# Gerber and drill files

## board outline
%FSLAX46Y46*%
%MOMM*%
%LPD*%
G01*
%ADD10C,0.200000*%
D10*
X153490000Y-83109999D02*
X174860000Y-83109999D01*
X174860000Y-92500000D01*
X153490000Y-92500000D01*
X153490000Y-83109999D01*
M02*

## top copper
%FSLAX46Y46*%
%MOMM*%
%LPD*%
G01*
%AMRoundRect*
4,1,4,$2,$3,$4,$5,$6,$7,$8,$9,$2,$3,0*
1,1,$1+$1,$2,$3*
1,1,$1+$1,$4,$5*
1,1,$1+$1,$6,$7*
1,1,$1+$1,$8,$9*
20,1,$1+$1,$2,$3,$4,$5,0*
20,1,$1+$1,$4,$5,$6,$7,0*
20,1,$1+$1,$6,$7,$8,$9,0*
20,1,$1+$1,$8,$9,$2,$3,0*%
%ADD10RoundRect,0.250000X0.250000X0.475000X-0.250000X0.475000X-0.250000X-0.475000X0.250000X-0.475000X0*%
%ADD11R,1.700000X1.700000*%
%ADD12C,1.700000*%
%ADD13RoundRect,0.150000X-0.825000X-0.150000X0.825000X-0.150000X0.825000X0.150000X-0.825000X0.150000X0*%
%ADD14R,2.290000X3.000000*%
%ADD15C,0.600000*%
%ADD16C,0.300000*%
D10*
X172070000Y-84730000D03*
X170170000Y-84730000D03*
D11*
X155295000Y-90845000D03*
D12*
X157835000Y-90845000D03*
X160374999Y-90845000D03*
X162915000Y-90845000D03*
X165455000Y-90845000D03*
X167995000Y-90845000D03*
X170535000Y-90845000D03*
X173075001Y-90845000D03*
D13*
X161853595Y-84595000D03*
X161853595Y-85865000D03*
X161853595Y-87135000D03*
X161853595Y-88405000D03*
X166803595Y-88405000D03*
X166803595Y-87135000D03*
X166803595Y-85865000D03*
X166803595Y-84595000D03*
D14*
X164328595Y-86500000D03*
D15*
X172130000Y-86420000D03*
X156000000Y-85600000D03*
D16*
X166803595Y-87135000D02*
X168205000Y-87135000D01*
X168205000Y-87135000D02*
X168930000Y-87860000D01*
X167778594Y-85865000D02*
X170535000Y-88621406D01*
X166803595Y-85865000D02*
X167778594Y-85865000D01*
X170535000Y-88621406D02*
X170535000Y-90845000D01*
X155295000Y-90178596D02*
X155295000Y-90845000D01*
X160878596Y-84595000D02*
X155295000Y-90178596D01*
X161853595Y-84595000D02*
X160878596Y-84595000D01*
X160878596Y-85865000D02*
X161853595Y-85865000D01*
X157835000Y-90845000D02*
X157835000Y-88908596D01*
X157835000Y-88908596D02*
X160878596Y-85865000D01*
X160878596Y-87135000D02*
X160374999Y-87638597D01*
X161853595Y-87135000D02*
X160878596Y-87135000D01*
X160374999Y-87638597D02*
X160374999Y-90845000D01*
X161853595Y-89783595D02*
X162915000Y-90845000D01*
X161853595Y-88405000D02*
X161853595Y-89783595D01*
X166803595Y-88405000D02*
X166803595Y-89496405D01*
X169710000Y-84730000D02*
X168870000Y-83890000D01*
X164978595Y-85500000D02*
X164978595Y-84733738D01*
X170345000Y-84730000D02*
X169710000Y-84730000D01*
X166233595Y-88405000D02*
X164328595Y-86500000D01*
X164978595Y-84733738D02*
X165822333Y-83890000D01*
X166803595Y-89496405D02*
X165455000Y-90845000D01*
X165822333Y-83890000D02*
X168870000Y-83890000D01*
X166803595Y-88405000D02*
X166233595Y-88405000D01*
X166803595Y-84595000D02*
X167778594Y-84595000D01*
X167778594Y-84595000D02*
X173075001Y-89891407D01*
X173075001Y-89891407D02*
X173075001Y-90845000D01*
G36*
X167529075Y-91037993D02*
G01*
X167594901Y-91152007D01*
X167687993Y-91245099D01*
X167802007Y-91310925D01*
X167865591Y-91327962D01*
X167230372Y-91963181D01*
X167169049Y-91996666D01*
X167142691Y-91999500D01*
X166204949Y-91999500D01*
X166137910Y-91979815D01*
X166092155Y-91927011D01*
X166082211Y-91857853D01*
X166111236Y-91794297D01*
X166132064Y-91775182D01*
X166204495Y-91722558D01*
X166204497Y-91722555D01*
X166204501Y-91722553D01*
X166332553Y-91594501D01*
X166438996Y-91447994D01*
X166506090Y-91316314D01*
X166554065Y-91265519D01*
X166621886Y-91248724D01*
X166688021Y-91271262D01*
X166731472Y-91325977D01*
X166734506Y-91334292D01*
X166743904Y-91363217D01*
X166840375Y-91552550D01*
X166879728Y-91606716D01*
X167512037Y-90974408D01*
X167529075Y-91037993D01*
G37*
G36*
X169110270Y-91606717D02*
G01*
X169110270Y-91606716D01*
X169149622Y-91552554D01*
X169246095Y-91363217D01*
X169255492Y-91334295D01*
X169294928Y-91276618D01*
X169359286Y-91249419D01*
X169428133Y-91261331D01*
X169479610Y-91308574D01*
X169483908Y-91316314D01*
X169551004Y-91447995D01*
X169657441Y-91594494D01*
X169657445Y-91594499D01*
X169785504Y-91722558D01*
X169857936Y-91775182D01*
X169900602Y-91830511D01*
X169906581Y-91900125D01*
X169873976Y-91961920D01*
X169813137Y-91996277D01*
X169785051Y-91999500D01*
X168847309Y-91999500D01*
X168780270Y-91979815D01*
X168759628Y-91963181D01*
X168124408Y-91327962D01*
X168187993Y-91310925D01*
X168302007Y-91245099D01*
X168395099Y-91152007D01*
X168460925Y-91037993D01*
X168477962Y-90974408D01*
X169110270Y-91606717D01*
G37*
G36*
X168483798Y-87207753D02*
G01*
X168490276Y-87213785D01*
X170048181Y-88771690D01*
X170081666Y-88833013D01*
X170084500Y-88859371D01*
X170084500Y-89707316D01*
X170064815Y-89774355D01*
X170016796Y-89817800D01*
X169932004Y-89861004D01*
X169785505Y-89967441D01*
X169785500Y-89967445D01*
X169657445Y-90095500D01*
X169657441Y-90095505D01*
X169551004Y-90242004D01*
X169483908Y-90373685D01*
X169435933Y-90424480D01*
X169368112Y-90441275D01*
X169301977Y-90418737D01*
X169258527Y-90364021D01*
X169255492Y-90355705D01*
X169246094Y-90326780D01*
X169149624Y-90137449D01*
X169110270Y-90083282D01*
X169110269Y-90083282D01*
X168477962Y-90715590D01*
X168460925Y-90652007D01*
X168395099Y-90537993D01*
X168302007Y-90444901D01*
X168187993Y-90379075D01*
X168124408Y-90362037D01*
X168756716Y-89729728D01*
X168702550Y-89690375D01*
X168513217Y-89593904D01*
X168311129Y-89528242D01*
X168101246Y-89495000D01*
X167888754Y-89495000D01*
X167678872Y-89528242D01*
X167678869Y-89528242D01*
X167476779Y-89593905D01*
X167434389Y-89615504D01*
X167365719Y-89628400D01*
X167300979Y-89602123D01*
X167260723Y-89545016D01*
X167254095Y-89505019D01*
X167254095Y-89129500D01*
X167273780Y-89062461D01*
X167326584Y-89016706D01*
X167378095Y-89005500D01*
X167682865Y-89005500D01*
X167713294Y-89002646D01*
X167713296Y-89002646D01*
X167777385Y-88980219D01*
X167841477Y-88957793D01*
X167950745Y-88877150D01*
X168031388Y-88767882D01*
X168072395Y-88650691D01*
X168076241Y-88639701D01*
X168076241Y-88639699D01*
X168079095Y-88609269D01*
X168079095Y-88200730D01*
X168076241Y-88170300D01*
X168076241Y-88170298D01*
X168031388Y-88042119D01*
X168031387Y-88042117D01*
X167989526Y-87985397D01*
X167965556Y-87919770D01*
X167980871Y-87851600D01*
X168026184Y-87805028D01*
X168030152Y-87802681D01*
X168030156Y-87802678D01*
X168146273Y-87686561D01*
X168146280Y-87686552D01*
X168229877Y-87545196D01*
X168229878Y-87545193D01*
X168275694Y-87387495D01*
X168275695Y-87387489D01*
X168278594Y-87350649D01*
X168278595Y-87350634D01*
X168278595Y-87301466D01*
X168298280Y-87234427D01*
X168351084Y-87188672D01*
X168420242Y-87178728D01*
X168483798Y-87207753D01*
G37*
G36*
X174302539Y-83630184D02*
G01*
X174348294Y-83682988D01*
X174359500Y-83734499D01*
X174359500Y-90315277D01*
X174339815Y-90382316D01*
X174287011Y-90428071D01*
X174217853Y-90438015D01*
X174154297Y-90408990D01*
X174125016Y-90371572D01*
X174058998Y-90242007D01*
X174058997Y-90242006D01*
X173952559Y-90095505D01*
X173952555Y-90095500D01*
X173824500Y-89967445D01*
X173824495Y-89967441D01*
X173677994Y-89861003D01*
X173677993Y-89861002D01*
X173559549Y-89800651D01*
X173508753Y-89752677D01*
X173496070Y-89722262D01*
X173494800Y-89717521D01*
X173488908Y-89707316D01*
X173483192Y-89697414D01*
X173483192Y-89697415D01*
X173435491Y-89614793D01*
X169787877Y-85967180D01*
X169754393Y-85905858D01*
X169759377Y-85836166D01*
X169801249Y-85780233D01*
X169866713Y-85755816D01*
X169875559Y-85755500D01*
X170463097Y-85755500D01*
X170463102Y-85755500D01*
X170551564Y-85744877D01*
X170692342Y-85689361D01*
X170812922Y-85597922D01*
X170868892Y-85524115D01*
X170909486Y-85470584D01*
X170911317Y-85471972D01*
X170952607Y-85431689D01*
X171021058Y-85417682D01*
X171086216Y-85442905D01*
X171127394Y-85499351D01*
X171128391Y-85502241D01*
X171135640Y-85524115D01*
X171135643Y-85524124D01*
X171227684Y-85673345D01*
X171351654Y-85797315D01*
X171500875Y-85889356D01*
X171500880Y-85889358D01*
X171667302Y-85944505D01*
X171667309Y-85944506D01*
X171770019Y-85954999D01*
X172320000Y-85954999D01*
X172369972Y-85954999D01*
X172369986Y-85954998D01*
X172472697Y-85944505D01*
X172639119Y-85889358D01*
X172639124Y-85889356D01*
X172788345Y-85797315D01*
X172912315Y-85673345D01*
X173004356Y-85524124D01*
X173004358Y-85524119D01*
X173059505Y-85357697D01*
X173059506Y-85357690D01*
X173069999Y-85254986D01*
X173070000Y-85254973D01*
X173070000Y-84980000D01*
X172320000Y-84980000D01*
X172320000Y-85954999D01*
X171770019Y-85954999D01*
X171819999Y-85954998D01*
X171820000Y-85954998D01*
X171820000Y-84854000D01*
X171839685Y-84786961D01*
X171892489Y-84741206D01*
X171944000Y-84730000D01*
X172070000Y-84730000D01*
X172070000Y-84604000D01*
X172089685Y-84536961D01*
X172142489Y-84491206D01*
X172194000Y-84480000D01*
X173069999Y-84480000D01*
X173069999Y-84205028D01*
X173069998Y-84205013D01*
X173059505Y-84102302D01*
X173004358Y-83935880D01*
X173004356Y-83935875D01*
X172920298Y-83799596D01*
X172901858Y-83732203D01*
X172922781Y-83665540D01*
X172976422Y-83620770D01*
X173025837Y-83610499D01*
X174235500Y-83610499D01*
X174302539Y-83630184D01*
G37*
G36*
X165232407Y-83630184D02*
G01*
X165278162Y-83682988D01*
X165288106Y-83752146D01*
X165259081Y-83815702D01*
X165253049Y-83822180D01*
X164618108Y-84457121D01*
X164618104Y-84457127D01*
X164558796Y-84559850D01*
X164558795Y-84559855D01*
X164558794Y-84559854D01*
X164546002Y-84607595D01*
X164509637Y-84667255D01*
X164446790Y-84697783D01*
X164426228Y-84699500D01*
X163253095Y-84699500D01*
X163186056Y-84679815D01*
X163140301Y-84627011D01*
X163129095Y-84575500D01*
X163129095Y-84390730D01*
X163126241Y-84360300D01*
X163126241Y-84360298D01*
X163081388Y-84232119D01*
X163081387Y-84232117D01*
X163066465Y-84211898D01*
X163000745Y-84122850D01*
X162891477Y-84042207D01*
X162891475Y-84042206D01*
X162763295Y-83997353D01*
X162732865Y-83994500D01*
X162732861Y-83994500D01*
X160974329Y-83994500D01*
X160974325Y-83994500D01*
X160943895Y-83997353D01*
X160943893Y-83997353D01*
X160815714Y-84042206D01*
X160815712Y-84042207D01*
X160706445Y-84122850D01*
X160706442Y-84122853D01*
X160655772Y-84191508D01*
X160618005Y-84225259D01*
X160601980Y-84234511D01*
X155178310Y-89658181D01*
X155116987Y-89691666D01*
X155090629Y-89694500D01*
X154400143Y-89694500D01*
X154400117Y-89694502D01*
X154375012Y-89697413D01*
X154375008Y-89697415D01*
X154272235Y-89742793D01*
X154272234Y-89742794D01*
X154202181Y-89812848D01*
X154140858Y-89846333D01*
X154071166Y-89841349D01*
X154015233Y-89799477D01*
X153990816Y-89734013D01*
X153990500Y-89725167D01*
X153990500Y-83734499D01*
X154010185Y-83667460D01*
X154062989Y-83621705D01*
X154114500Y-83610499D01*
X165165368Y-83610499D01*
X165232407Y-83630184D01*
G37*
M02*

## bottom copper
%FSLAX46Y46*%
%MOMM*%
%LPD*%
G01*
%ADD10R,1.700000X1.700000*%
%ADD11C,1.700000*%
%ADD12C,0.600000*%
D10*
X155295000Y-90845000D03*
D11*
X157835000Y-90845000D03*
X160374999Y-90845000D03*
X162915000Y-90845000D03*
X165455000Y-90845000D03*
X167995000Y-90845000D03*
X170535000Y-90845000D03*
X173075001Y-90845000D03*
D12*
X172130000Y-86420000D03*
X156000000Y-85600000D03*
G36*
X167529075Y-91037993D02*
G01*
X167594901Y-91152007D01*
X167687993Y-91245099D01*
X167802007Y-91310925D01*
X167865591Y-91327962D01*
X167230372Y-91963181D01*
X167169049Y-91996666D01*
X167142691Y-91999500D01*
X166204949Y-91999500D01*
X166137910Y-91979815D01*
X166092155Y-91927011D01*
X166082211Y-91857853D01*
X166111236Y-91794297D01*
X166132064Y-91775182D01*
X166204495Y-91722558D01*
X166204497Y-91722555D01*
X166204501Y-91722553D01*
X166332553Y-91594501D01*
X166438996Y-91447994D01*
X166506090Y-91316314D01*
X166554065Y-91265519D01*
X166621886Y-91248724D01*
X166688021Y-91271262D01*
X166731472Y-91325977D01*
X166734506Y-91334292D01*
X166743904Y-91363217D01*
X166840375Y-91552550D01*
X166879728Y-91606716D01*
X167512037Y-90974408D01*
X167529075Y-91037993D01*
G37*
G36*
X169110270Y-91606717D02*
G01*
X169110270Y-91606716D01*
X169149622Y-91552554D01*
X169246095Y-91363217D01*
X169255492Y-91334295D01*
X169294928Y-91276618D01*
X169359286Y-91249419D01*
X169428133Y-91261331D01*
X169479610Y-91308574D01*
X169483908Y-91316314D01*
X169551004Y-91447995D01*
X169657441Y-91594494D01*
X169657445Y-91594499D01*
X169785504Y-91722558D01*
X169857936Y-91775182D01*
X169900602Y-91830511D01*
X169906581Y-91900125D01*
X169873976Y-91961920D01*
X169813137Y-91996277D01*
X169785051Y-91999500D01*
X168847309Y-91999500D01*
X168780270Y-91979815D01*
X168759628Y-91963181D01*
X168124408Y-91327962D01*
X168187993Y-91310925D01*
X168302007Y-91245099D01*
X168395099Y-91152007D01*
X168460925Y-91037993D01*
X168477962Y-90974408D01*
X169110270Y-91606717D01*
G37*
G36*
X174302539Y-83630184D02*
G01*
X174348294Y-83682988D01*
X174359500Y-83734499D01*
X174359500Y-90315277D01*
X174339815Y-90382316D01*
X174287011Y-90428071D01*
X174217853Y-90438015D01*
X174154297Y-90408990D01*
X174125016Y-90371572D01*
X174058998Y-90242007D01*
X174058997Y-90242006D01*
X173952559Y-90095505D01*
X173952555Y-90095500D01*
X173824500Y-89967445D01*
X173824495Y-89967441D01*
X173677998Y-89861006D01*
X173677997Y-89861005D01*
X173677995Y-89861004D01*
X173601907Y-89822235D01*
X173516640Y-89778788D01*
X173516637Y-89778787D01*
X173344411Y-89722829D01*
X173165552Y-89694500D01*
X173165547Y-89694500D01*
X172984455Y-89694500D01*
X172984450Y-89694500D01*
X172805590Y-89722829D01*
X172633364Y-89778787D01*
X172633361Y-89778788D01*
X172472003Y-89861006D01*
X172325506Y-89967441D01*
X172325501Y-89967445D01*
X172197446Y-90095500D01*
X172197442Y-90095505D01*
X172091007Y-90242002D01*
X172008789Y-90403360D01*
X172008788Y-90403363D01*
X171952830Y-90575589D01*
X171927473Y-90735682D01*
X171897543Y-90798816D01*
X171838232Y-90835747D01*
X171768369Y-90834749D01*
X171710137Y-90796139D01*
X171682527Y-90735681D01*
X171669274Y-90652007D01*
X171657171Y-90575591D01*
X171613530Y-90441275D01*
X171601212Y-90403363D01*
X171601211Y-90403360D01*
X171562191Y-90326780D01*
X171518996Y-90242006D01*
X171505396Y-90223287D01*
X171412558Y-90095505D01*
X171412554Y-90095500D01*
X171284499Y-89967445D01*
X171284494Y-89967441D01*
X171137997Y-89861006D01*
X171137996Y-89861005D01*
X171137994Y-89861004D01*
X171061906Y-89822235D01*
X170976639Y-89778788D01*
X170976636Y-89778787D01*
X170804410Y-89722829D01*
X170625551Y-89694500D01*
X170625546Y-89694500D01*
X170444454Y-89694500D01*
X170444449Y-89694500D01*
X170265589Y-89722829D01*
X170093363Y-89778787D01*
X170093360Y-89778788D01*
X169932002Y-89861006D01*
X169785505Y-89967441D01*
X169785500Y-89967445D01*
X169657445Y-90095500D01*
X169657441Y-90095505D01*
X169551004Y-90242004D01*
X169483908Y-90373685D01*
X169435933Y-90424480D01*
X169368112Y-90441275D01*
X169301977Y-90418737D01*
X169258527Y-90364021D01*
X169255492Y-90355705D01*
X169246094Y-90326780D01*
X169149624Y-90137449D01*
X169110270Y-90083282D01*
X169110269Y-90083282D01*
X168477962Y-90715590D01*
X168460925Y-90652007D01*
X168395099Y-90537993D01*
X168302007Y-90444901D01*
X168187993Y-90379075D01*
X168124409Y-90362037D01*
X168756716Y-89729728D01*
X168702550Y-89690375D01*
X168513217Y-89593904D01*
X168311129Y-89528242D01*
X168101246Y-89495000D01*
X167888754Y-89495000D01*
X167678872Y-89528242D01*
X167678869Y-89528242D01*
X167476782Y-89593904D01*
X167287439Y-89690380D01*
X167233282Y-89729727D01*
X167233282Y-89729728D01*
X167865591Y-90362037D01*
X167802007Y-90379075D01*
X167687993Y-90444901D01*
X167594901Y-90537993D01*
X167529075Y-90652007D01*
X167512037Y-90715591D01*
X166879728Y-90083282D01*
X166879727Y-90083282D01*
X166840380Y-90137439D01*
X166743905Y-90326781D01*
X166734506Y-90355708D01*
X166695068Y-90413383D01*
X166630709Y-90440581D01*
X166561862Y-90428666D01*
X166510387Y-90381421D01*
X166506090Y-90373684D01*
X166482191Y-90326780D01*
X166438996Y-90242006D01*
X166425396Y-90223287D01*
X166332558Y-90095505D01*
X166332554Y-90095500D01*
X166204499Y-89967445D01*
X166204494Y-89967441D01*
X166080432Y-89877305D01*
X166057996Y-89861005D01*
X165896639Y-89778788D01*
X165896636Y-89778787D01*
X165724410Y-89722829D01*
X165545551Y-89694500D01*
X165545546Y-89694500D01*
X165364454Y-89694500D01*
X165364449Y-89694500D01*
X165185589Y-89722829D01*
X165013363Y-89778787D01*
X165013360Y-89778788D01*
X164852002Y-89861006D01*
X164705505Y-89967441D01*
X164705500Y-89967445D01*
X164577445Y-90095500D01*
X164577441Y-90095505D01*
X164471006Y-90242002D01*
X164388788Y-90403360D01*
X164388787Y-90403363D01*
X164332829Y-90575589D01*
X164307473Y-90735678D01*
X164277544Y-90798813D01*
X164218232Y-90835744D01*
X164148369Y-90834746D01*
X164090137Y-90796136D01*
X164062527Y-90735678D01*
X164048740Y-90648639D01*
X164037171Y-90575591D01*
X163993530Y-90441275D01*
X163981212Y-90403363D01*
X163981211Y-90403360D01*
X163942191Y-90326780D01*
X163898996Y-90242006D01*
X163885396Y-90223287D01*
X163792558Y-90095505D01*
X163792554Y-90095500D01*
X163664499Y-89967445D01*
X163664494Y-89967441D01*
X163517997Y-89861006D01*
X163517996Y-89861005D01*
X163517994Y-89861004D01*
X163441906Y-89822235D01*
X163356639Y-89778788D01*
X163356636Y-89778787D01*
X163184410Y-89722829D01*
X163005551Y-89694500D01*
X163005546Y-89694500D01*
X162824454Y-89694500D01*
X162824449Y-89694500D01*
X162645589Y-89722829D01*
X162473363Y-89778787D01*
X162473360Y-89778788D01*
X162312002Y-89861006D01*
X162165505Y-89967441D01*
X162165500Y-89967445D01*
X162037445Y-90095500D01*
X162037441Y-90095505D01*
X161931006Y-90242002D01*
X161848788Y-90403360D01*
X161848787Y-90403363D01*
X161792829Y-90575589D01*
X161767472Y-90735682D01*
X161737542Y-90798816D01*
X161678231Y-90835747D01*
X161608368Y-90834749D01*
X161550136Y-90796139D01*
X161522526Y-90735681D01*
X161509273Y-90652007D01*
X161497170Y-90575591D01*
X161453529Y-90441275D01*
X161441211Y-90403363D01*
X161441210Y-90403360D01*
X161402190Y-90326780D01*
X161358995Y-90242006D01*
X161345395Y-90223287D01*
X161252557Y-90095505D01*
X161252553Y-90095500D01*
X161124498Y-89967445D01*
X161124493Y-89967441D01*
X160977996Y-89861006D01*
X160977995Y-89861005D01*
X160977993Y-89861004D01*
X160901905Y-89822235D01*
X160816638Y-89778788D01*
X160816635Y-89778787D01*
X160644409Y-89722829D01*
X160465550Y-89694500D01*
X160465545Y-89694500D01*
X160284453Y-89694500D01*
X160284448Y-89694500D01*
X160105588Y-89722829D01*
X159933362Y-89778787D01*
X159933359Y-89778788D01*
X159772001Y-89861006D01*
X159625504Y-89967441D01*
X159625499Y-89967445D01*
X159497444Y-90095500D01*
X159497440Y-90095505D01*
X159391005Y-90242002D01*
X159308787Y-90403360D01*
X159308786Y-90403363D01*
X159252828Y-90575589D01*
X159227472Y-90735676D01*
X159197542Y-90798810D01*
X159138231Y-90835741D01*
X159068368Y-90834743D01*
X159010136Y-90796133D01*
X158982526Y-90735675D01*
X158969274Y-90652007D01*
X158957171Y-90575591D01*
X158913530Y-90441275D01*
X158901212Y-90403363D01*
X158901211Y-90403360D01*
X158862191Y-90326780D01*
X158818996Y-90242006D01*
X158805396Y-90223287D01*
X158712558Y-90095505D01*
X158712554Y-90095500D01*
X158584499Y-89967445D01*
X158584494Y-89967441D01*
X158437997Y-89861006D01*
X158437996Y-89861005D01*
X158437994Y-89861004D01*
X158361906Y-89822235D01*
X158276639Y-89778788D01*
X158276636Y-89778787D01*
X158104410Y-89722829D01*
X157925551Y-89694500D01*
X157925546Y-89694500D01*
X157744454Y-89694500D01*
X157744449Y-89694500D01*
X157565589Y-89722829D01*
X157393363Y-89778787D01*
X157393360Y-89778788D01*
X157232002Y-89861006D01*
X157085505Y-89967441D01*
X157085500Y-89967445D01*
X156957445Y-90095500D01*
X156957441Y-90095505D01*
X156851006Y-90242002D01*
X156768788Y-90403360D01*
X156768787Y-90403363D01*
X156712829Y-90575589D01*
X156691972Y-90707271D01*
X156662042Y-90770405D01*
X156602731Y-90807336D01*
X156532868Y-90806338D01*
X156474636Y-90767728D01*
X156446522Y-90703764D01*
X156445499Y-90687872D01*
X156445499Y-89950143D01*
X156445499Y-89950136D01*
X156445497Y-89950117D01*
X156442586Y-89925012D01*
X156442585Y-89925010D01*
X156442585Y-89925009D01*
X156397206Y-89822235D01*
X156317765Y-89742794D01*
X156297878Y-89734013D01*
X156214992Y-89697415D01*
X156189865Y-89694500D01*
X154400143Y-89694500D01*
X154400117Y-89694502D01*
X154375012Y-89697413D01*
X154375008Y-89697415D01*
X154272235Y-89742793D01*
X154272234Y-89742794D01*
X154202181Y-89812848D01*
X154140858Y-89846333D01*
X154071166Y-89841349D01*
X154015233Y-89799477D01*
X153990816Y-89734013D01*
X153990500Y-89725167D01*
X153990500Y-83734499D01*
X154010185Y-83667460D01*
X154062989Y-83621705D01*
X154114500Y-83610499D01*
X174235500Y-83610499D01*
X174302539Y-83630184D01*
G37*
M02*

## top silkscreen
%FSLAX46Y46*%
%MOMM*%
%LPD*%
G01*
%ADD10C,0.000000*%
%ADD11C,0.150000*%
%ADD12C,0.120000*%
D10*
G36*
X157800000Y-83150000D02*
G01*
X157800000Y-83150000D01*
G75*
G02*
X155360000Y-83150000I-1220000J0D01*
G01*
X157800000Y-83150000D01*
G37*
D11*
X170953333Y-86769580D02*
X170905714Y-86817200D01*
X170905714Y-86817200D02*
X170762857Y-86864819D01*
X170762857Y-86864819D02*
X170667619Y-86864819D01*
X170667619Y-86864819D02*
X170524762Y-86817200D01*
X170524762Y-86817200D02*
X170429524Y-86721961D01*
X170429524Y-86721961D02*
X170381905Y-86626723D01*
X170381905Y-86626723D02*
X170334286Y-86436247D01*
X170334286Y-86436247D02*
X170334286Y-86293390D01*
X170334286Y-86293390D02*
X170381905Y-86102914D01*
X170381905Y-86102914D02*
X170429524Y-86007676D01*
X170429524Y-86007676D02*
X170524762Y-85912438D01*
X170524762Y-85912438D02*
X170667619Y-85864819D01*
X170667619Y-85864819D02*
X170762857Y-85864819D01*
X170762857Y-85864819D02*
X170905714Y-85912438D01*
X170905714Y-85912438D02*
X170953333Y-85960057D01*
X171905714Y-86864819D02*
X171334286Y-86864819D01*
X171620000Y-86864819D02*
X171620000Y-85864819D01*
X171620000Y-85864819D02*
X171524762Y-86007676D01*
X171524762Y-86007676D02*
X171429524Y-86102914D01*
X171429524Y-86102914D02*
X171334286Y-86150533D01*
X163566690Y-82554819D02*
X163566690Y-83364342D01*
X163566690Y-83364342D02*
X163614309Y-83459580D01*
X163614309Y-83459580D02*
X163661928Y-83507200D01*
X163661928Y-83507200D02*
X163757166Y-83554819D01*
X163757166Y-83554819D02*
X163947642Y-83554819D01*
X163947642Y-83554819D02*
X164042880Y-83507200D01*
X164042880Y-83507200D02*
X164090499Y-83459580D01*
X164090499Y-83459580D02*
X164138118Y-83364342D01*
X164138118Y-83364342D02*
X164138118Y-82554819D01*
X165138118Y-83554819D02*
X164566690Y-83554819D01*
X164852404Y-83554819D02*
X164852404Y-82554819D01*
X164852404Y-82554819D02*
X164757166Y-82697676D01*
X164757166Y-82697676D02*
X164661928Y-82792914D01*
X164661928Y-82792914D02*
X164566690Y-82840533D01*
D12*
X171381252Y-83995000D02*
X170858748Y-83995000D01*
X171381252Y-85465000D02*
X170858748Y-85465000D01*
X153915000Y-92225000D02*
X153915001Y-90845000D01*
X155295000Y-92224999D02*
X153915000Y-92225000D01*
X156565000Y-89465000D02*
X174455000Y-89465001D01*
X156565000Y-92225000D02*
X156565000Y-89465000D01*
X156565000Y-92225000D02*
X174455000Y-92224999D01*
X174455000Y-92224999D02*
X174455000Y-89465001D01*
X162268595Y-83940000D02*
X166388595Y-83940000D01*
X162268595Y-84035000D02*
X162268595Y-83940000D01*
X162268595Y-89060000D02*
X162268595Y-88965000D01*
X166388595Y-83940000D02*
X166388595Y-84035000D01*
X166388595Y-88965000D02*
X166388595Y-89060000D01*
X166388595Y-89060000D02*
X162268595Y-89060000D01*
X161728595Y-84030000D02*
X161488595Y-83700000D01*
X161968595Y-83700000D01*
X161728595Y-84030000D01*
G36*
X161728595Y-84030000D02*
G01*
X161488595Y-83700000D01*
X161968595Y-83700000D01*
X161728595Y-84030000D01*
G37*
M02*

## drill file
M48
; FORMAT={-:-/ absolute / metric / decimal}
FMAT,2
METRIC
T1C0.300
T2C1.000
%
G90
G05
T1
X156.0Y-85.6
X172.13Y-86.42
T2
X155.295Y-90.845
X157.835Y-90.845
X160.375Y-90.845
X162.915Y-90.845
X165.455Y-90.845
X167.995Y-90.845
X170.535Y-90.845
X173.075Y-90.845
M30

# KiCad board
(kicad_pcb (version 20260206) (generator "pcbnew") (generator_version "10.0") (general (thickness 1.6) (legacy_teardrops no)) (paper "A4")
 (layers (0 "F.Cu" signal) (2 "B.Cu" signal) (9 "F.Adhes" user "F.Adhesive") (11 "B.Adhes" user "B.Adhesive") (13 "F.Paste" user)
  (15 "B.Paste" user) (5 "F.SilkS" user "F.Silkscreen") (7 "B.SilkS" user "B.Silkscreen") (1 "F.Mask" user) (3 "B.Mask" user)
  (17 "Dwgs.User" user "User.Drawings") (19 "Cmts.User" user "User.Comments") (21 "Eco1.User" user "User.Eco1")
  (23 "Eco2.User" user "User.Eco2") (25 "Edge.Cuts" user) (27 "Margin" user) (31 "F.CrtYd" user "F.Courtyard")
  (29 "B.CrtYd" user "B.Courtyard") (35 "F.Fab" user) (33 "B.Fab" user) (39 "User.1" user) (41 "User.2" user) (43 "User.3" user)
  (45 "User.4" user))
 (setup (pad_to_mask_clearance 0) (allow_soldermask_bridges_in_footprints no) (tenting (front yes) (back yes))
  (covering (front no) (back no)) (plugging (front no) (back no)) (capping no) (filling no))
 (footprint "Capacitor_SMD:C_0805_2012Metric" (layer "F.Cu") (at 171.12 84.73 180)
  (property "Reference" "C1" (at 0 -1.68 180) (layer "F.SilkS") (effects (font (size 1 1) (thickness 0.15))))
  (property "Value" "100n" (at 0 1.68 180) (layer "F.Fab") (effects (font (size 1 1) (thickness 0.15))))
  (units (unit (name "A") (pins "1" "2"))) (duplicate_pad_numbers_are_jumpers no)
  (fp_line (start -0.261252 0.735) (end 0.261252 0.735) (stroke (width 0.12) (type solid)) (layer "F.SilkS"))
  (fp_line (start -0.261252 -0.735) (end 0.261252 -0.735) (stroke (width 0.12) (type solid)) (layer "F.SilkS"))
  (pad "1" smd roundrect (at -0.95 0 180) (size 1 1.45) (layers "F.Cu" "F.Mask" "F.Paste") (roundrect_rratio 0.25) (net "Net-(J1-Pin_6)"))
  (pad "2" smd roundrect (at 0.95 0 180) (size 1 1.45) (layers "F.Cu" "F.Mask" "F.Paste") (roundrect_rratio 0.25) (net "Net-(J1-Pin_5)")))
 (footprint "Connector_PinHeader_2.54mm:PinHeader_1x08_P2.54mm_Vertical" (layer "F.Cu") (at 155.295 90.845 90)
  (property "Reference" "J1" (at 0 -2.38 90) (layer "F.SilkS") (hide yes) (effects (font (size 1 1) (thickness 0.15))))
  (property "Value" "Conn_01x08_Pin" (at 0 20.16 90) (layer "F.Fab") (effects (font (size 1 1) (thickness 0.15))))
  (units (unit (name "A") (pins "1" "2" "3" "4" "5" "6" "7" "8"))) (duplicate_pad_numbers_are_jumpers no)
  (fp_line (start -1.38 -1.38) (end 0 -1.379999) (stroke (width 0.12) (type solid)) (layer "F.SilkS"))
  (fp_line (start -1.379999 0) (end -1.38 -1.38) (stroke (width 0.12) (type solid)) (layer "F.SilkS"))
  (fp_line (start 1.38 1.27) (end 1.379999 19.16) (stroke (width 0.12) (type solid)) (layer "F.SilkS"))
  (fp_line (start -1.38 1.27) (end 1.38 1.27) (stroke (width 0.12) (type solid)) (layer "F.SilkS"))
  (fp_line (start -1.38 1.27) (end -1.379999 19.16) (stroke (width 0.12) (type solid)) (layer "F.SilkS"))
  (fp_line (start -1.379999 19.16) (end 1.379999 19.16) (stroke (width 0.12) (type solid)) (layer "F.SilkS"))
  (pad "1" thru_hole rect (at 0 0 90) (size 1.7 1.7) (drill 1) (layers "*.Cu" "*.Mask") (remove_unused_layers no) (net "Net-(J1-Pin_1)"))
  (pad "2" thru_hole circle (at 0 2.54 90) (size 1.7 1.7) (drill 1) (layers "*.Cu" "*.Mask") (remove_unused_layers no)
   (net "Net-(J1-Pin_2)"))
  (pad "3" thru_hole circle (at 0 5.079999 90) (size 1.7 1.7) (drill 1) (layers "*.Cu" "*.Mask") (remove_unused_layers no)
   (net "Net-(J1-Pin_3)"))
  (pad "4" thru_hole circle (at 0 7.62 90) (size 1.7 1.7) (drill 1) (layers "*.Cu" "*.Mask") (remove_unused_layers no)
   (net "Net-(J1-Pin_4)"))
  (pad "5" thru_hole circle (at 0 10.16 90) (size 1.7 1.7) (drill 1) (layers "*.Cu" "*.Mask") (remove_unused_layers no)
   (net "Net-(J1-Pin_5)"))
  (pad "6" thru_hole circle (at 0 12.7 90) (size 1.7 1.7) (drill 1) (layers "*.Cu" "*.Mask") (remove_unused_layers no)
   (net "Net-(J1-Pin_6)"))
  (pad "7" thru_hole circle (at 0 15.24 90) (size 1.7 1.7) (drill 1) (layers "*.Cu" "*.Mask") (remove_unused_layers no)
   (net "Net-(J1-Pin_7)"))
  (pad "8" thru_hole circle (at 0 17.780001 90) (size 1.7 1.7) (drill 1) (layers "*.Cu" "*.Mask") (remove_unused_layers no)
   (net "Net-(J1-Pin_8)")))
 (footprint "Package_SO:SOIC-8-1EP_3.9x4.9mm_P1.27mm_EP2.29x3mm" (layer "F.Cu") (at 164.328595 86.5)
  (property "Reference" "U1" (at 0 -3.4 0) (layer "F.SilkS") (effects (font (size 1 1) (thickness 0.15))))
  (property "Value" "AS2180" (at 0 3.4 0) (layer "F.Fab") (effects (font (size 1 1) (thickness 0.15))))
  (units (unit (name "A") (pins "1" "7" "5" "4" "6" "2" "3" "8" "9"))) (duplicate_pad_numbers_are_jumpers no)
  (fp_line (start -2.06 -2.56) (end 2.06 -2.56) (stroke (width 0.12) (type solid)) (layer "F.SilkS"))
  (fp_line (start -2.06 -2.465) (end -2.06 -2.56) (stroke (width 0.12) (type solid)) (layer "F.SilkS"))
  (fp_line (start -2.06 2.56) (end -2.06 2.465) (stroke (width 0.12) (type solid)) (layer "F.SilkS"))
  (fp_line (start 2.06 -2.56) (end 2.06 -2.465) (stroke (width 0.12) (type solid)) (layer "F.SilkS"))
  (fp_line (start 2.06 2.465) (end 2.06 2.56) (stroke (width 0.12) (type solid)) (layer "F.SilkS"))
  (fp_line (start 2.06 2.56) (end -2.06 2.56) (stroke (width 0.12) (type solid)) (layer "F.SilkS"))
  (fp_poly (pts (xy -2.6 -2.47) (xy -2.84 -2.8) (xy -2.36 -2.8)) (stroke (width 0.12) (type solid)) (fill yes) (layer "F.SilkS"))
  (pad "" smd roundrect (at -0.57 -0.75) (size 0.92 1.21) (layers "F.Paste") (roundrect_rratio 0.25))
  (pad "" smd roundrect (at -0.57 0.75) (size 0.92 1.21) (layers "F.Paste") (roundrect_rratio 0.25))
  (pad "" smd roundrect (at 0.57 -0.75) (size 0.92 1.21) (layers "F.Paste") (roundrect_rratio 0.25))
  (pad "" smd roundrect (at 0.57 0.75) (size 0.92 1.21) (layers "F.Paste") (roundrect_rratio 0.25))
  (pad "1" smd roundrect (at -2.475 -1.905) (size 1.95 0.6) (layers "F.Cu" "F.Mask" "F.Paste") (roundrect_rratio 0.25)
   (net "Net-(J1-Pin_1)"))
  (pad "2" smd roundrect (at -2.475 -0.635) (size 1.95 0.6) (layers "F.Cu" "F.Mask" "F.Paste") (roundrect_rratio 0.25)
   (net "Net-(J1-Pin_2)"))
  (pad "3" smd roundrect (at -2.475 0.635) (size 1.95 0.6) (layers "F.Cu" "F.Mask" "F.Paste") (roundrect_rratio 0.25) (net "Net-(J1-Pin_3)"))
  (pad "4" smd roundrect (at -2.475 1.905) (size 1.95 0.6) (layers "F.Cu" "F.Mask" "F.Paste") (roundrect_rratio 0.25) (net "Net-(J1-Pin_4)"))
  (pad "5" smd roundrect (at 2.475 1.905) (size 1.95 0.6) (layers "F.Cu" "F.Mask" "F.Paste") (roundrect_rratio 0.25) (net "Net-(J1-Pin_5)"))
  (pad "6" smd roundrect (at 2.475 0.635) (size 1.95 0.6) (layers "F.Cu" "F.Mask" "F.Paste") (roundrect_rratio 0.25) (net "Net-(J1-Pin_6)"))
  (pad "7" smd roundrect (at 2.475 -0.635) (size 1.95 0.6) (layers "F.Cu" "F.Mask" "F.Paste") (roundrect_rratio 0.25) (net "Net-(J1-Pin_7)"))
  (pad "8" smd roundrect (at 2.475 -1.905) (size 1.95 0.6) (layers "F.Cu" "F.Mask" "F.Paste") (roundrect_rratio 0.25) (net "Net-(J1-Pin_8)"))
  (pad "9" smd rect (at 0 0) (size 2.29 3) (layers "F.Cu" "F.Mask") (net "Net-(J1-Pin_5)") (zone_connect 2)))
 (gr_poly
  (pts (arc (start 155.36 83.15) (mid 156.58 84.37) (end 157.8 83.15))) (stroke (width 0) (type solid)) (fill yes) (layer "F.SilkS"))
 (gr_rect (start 153.49 83.109999) (end 174.86 92.5) (stroke (width 0.2) (type solid)) (fill no) (layer "Edge.Cuts"))
 (segment (start 166.803595 87.135) (end 168.205 87.135) (width 0.3) (layer "F.Cu") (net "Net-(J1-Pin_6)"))
 (segment (start 168.205 87.135) (end 168.93 87.86) (width 0.3) (layer "F.Cu") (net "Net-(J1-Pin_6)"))
 (via (at 172.13 86.42) (size 0.6) (drill 0.3) (layers "F.Cu" "B.Cu") (free yes) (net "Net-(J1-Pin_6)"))
 (via (at 156 85.6) (size 0.6) (drill 0.3) (layers "F.Cu" "B.Cu") (free yes) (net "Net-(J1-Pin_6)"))
 (segment (start 167.778594 85.865) (end 170.535 88.621406) (width 0.3) (layer "F.Cu") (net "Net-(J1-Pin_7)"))
 (segment (start 166.803595 85.865) (end 167.778594 85.865) (width 0.3) (layer "F.Cu") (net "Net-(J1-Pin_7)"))
 (segment (start 170.535 88.621406) (end 170.535 90.845) (width 0.3) (layer "F.Cu") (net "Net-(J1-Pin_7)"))
 (segment (start 155.295 90.178596) (end 155.295 90.845) (width 0.3) (layer "F.Cu") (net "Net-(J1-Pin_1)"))
 (segment (start 160.878596 84.595) (end 155.295 90.178596) (width 0.3) (layer "F.Cu") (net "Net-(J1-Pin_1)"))
 (segment (start 161.853595 84.595) (end 160.878596 84.595) (width 0.3) (layer "F.Cu") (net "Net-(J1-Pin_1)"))
 (segment (start 160.878596 85.865) (end 161.853595 85.865) (width 0.3) (layer "F.Cu") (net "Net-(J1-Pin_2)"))
 (segment (start 157.835 90.845) (end 157.835 88.908596) (width 0.3) (layer "F.Cu") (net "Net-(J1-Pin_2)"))
 (segment (start 157.835 88.908596) (end 160.878596 85.865) (width 0.3) (layer "F.Cu") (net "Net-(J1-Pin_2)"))
 (segment (start 160.878596 87.135) (end 160.374999 87.638597) (width 0.3) (layer "F.Cu") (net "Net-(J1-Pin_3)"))
 (segment (start 161.853595 87.135) (end 160.878596 87.135) (width 0.3) (layer "F.Cu") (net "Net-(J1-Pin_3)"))
 (segment (start 160.374999 87.638597) (end 160.374999 90.845) (width 0.3) (layer "F.Cu") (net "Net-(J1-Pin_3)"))
 (segment (start 161.853595 89.783595) (end 162.915 90.845) (width 0.3) (layer "F.Cu") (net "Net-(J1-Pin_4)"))
 (segment (start 161.853595 88.405) (end 161.853595 89.783595) (width 0.3) (layer "F.Cu") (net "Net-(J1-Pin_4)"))
 (segment (start 166.803595 88.405) (end 166.803595 89.496405) (width 0.3) (layer "F.Cu") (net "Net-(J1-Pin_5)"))
 (segment (start 169.71 84.73) (end 168.87 83.89) (width 0.3) (layer "F.Cu") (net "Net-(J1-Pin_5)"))
 (segment (start 164.978595 85.5) (end 164.978595 84.733738) (width 0.3) (layer "F.Cu") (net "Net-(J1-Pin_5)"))
 (segment (start 170.345 84.73) (end 169.71 84.73) (width 0.3) (layer "F.Cu") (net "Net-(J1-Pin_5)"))
 (segment (start 166.233595 88.405) (end 164.328595 86.5) (width 0.3) (layer "F.Cu") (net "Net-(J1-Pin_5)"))
 (segment (start 164.978595 84.733738) (end 165.822333 83.89) (width 0.3) (layer "F.Cu") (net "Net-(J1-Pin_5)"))
 (segment (start 166.803595 89.496405) (end 165.455 90.845) (width 0.3) (layer "F.Cu") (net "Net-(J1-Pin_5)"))
 (segment (start 165.822333 83.89) (end 168.87 83.89) (width 0.3) (layer "F.Cu") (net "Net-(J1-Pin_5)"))
 (segment (start 166.803595 88.405) (end 166.233595 88.405) (width 0.3) (layer "F.Cu") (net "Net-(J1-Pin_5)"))
 (segment (start 166.803595 84.595) (end 167.778594 84.595) (width 0.3) (layer "F.Cu") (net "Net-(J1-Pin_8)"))
 (segment (start 167.778594 84.595) (end 173.075001 89.891407) (width 0.3) (layer "F.Cu") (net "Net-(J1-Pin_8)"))
 (segment (start 173.075001 89.891407) (end 173.075001 90.845) (width 0.3) (layer "F.Cu") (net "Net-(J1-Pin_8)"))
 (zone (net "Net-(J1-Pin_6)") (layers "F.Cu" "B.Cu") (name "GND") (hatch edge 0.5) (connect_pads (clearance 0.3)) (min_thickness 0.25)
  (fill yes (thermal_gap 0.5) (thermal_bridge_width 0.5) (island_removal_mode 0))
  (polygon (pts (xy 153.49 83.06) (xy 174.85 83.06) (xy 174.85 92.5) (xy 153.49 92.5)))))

